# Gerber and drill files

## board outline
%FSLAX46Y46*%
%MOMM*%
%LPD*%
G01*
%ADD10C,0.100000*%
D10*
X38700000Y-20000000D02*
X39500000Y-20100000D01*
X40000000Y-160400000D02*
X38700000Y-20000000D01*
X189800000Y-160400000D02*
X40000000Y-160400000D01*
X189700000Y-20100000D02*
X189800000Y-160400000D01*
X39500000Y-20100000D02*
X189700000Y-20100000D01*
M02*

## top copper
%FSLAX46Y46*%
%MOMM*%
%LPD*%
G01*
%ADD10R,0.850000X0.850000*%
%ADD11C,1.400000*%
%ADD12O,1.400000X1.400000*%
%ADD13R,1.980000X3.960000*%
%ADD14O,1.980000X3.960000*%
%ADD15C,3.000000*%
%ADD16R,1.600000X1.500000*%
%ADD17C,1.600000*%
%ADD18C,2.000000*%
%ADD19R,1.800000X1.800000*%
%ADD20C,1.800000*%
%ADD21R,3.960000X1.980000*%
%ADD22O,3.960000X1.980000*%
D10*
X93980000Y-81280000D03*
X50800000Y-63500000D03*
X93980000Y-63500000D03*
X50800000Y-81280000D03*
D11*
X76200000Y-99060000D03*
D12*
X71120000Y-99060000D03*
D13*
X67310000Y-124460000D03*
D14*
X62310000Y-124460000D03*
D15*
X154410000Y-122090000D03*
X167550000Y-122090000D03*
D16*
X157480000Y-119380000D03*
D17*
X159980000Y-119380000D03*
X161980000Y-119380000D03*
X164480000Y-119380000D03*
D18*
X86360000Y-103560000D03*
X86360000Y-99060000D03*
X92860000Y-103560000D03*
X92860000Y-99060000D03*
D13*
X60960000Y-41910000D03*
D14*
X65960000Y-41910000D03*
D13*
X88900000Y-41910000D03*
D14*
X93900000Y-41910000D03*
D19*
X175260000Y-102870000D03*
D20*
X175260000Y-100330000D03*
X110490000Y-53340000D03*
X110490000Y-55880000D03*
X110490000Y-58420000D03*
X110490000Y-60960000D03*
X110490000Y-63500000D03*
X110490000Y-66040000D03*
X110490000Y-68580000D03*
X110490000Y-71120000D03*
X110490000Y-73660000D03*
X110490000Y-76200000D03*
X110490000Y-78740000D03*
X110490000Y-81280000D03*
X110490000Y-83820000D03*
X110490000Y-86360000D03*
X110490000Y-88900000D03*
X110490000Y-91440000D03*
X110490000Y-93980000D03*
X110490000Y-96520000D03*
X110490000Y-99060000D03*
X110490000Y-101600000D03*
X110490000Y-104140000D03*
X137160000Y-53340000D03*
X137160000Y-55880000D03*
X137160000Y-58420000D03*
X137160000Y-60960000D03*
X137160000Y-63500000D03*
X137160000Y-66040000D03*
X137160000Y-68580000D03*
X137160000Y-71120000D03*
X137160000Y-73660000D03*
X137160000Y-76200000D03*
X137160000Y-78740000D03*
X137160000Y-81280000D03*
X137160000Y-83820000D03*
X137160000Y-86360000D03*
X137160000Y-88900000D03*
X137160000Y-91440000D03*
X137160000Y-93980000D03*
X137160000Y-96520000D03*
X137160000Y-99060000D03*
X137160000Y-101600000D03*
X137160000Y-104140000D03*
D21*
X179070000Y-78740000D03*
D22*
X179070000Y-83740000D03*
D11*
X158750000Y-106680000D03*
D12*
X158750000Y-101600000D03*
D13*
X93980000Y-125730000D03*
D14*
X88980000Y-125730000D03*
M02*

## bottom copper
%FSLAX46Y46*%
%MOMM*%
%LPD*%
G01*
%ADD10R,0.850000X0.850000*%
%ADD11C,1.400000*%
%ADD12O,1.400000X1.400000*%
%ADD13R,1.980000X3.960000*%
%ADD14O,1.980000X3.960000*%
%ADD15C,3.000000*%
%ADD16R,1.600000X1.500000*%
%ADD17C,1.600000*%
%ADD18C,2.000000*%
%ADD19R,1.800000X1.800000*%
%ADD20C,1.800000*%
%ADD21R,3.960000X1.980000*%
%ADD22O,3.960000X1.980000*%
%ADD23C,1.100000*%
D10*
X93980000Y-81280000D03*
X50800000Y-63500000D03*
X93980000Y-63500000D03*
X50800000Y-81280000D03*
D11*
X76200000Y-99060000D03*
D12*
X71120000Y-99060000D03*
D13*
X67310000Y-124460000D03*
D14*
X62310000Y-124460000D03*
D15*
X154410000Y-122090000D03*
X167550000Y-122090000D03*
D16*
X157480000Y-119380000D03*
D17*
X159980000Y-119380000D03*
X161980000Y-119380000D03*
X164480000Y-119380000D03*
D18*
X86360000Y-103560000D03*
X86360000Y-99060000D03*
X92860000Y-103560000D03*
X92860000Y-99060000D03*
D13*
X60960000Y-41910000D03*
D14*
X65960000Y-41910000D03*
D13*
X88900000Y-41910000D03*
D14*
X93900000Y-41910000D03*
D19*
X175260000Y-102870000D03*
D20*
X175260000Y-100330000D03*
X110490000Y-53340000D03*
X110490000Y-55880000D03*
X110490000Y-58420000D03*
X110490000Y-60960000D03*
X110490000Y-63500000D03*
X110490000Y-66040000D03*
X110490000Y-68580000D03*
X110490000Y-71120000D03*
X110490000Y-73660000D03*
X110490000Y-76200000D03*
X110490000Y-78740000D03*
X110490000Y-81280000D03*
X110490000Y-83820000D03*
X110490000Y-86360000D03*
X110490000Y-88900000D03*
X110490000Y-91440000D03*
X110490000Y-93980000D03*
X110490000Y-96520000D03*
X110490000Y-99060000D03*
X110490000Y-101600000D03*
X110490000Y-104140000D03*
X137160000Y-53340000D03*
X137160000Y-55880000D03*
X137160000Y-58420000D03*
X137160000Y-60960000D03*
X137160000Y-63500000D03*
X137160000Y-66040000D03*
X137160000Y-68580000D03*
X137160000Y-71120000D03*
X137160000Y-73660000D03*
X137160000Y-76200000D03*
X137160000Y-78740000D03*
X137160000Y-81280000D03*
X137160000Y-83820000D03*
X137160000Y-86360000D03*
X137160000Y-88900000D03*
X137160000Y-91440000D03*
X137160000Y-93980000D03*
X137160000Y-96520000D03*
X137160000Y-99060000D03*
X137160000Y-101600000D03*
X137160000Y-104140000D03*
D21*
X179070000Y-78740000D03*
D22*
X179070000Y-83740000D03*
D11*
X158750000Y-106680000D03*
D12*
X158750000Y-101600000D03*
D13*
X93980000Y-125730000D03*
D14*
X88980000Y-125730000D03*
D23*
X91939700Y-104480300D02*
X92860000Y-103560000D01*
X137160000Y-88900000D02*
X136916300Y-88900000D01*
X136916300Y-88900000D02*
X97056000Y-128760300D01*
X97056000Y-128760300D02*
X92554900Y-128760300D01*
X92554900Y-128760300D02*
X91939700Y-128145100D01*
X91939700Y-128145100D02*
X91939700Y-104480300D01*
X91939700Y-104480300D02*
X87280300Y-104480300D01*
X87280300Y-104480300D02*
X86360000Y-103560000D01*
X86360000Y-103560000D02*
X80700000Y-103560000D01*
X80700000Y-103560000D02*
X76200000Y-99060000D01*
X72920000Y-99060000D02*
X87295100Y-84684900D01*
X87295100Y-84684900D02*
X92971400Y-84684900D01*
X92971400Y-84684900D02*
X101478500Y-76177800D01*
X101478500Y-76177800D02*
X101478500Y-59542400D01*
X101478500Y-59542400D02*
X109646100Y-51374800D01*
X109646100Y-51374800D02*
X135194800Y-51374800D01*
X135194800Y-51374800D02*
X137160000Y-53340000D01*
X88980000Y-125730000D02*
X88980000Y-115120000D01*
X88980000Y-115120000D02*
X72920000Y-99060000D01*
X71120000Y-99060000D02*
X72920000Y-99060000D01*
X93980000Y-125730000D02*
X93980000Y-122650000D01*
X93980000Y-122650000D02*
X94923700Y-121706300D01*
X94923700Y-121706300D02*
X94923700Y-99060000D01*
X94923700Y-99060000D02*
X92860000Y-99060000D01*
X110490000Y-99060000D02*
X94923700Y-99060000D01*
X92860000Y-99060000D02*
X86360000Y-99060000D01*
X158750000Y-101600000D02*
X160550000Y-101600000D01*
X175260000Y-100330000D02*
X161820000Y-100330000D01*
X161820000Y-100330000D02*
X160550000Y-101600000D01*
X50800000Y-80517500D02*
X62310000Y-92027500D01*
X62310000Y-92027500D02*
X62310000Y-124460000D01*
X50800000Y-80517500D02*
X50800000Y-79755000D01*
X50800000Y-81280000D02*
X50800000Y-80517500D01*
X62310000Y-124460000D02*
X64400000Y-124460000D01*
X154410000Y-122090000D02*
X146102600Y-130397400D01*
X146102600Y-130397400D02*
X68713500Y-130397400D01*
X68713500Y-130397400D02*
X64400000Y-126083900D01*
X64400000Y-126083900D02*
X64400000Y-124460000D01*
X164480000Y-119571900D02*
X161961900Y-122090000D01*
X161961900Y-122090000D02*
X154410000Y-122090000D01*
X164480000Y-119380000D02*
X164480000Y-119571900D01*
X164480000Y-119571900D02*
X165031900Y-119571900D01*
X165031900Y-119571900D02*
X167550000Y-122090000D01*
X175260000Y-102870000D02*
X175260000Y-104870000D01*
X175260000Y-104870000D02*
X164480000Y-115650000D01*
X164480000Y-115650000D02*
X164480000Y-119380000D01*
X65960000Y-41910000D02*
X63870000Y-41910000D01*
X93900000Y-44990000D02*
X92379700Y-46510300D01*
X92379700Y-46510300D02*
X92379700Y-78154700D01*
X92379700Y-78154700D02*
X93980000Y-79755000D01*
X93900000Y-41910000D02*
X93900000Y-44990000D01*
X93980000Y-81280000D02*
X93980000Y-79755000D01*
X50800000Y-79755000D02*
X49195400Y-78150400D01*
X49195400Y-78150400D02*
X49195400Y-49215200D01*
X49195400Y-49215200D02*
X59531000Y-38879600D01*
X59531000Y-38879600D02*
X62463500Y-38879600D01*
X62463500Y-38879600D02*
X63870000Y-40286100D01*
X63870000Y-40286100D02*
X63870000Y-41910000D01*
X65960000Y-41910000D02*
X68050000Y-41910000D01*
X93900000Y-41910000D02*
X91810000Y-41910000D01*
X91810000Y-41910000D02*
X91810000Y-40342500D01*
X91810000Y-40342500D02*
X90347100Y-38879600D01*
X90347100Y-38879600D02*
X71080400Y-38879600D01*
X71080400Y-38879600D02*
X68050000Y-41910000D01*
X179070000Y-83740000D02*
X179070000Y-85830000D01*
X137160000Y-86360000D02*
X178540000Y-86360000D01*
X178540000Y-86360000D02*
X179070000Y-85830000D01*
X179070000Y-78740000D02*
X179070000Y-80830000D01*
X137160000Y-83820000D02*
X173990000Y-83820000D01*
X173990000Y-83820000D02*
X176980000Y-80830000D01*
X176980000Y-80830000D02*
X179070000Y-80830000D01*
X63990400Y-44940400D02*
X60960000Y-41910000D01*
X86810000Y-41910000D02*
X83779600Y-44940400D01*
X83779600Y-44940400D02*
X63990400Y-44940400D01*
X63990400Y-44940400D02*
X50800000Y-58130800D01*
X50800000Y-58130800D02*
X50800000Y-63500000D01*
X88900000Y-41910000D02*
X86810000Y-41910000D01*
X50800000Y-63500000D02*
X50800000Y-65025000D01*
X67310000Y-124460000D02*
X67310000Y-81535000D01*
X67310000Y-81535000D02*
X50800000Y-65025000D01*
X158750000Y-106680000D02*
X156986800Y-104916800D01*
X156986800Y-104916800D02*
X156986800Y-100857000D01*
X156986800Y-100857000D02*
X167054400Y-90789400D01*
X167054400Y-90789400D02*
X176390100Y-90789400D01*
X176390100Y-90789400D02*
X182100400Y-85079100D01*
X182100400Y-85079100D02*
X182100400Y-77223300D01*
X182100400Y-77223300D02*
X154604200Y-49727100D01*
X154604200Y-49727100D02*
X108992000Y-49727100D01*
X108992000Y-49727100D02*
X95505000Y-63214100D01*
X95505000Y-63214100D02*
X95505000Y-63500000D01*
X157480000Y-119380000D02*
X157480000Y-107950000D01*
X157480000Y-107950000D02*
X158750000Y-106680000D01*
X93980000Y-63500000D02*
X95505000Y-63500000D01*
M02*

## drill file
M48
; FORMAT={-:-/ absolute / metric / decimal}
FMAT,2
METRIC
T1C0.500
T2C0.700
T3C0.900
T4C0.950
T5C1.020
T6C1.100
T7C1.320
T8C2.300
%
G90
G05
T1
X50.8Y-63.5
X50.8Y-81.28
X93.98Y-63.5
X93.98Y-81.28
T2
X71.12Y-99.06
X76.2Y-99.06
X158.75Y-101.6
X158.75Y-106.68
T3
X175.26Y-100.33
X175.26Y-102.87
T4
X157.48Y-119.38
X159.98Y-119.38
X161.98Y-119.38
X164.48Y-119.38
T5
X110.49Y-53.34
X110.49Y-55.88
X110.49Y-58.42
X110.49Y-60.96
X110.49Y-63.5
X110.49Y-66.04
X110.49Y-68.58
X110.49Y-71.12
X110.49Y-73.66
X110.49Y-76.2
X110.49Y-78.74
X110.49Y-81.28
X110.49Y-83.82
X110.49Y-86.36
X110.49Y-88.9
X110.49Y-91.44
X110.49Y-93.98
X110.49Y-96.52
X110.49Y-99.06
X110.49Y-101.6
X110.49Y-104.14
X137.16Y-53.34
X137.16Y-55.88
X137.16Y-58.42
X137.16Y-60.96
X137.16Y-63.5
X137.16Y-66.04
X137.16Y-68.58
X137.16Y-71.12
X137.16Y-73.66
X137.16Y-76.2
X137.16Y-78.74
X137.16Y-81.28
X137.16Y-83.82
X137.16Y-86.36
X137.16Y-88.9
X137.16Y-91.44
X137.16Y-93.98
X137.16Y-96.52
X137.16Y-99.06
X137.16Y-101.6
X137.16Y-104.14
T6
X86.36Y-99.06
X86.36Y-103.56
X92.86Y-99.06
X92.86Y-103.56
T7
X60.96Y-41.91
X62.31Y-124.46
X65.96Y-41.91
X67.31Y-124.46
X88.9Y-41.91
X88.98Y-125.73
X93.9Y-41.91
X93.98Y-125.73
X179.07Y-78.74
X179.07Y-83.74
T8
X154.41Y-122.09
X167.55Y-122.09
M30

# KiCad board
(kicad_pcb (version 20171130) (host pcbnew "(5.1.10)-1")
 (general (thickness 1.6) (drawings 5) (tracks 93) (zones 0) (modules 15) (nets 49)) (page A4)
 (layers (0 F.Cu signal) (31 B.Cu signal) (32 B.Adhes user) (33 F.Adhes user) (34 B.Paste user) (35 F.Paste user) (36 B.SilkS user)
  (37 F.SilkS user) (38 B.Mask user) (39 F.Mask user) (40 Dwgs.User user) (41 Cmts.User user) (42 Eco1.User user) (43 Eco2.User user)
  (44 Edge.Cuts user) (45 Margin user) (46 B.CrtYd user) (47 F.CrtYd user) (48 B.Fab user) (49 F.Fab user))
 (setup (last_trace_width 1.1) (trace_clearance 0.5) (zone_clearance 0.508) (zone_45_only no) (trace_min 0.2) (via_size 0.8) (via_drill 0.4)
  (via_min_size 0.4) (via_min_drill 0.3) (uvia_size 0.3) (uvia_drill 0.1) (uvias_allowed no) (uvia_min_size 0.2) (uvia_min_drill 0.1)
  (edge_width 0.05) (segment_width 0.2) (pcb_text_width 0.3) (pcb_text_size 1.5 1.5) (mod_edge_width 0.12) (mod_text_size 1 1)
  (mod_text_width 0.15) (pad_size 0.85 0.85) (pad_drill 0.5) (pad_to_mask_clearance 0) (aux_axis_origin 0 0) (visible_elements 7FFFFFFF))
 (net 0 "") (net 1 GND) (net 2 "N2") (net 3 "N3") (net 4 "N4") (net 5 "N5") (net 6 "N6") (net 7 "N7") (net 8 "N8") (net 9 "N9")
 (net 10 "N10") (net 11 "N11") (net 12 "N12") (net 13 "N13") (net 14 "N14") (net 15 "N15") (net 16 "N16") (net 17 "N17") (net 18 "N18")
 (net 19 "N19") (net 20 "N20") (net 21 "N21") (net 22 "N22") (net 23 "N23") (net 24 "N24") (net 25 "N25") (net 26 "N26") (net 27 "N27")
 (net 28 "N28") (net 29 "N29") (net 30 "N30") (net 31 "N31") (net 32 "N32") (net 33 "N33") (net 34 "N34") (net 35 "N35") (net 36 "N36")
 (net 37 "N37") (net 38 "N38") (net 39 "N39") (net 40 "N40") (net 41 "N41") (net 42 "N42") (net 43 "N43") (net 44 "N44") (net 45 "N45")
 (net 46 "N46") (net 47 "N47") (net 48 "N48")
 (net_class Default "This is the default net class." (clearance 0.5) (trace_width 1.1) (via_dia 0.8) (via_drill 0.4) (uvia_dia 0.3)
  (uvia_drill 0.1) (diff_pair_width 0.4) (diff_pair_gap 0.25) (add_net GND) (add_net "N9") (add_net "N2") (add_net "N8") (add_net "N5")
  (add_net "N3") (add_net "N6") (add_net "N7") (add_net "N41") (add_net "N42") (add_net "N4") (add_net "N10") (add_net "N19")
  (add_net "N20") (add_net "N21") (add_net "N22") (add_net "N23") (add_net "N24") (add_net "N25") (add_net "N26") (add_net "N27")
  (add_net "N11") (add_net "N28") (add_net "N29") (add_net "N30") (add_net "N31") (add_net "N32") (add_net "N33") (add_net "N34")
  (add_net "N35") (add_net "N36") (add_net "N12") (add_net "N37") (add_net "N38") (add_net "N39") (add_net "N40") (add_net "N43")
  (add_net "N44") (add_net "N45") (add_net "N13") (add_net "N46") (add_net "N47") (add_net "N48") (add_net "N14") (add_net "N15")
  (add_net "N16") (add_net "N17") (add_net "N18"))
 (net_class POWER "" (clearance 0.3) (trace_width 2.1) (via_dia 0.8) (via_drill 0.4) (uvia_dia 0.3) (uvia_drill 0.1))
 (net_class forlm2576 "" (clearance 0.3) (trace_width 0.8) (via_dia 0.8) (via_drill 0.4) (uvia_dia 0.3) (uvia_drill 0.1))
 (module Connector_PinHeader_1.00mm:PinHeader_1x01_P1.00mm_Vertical (layer F.Cu) (at 93.98 81.28)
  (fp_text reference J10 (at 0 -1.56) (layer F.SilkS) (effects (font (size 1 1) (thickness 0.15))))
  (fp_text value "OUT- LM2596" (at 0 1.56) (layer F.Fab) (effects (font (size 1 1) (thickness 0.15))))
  (pad 1 thru_hole rect (at 0 0) (size 0.85 0.85) (drill 0.5) (layers *.Cu *.Mask) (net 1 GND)))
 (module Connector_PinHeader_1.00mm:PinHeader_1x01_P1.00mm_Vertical (layer F.Cu) (at 50.8 63.5)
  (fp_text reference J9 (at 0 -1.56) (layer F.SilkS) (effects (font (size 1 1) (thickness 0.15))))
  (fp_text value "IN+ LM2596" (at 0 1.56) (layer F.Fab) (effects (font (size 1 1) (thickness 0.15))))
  (pad 1 thru_hole rect (at 0 0) (size 0.85 0.85) (drill 0.5) (layers *.Cu *.Mask) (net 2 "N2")))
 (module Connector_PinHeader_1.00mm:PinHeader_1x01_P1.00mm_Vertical (layer F.Cu) (at 93.98 63.5)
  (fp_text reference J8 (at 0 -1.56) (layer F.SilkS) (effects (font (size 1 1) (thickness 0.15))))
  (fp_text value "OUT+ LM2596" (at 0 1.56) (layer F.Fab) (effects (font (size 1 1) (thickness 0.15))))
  (pad 1 thru_hole rect (at 0 0) (size 0.85 0.85) (drill 0.5) (layers *.Cu *.Mask) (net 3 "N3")))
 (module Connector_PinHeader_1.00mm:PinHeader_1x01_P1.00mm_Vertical (layer F.Cu) (at 50.8 81.28)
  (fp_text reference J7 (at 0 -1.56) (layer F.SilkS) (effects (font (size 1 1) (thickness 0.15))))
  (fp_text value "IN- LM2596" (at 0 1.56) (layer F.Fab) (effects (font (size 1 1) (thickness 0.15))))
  (pad 1 thru_hole rect (at 0 0) (size 0.85 0.85) (drill 0.5) (layers *.Cu *.Mask) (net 1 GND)))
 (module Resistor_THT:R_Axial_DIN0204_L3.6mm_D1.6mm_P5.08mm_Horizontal (layer F.Cu) (at 76.2 99.06 180)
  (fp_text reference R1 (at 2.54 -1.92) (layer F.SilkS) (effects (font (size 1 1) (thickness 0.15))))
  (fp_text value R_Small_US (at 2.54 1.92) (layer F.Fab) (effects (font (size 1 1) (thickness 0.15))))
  (pad 1 thru_hole circle (at 0 0 180) (size 1.4 1.4) (drill 0.7) (layers *.Cu *.Mask) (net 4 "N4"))
  (pad 2 thru_hole oval (at 5.08 0 180) (size 1.4 1.4) (drill 0.7) (layers *.Cu *.Mask) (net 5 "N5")))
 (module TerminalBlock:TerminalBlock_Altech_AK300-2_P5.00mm (layer F.Cu) (at 67.31 124.46 180)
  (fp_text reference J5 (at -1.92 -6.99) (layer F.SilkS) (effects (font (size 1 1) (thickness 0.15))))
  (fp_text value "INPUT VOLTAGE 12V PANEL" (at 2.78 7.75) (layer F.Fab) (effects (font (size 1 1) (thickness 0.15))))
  (pad 1 thru_hole rect (at 0 0 180) (size 1.98 3.96) (drill 1.32) (layers *.Cu *.Mask) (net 2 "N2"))
  (pad 2 thru_hole oval (at 5 0 180) (size 1.98 3.96) (drill 1.32) (layers *.Cu *.Mask) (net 1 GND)))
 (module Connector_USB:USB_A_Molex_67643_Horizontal (layer F.Cu) (at 157.48 119.38)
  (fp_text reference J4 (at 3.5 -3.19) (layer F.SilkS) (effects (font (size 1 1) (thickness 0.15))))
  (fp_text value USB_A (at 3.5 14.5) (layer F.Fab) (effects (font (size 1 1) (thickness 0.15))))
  (pad 5 thru_hole circle (at -3.07 2.71) (size 3 3) (drill 2.3) (layers *.Cu *.Mask) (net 1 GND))
  (pad 5 thru_hole circle (at 10.07 2.71) (size 3 3) (drill 2.3) (layers *.Cu *.Mask) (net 1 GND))
  (pad 1 thru_hole rect (at 0 0) (size 1.6 1.5) (drill 0.95) (layers *.Cu *.Mask) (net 3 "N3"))
  (pad 2 thru_hole circle (at 2.5 0) (size 1.6 1.6) (drill 0.95) (layers *.Cu *.Mask) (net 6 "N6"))
  (pad 3 thru_hole circle (at 4.5 0) (size 1.6 1.6) (drill 0.95) (layers *.Cu *.Mask) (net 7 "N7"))
  (pad 4 thru_hole circle (at 7 0) (size 1.6 1.6) (drill 0.95) (layers *.Cu *.Mask) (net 1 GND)))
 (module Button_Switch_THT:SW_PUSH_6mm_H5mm (layer F.Cu) (at 86.36 99.06)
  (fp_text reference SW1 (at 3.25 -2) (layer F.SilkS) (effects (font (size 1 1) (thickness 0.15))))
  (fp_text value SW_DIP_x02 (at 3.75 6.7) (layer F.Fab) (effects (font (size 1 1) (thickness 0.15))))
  (pad 2 thru_hole circle (at 0 4.5 90) (size 2 2) (drill 1.1) (layers *.Cu *.Mask) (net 4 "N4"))
  (pad 1 thru_hole circle (at 0 0 90) (size 2 2) (drill 1.1) (layers *.Cu *.Mask) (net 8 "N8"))
  (pad 2 thru_hole circle (at 6.5 4.5 90) (size 2 2) (drill 1.1) (layers *.Cu *.Mask) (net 4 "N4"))
  (pad 1 thru_hole circle (at 6.5 0 90) (size 2 2) (drill 1.1) (layers *.Cu *.Mask) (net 8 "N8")))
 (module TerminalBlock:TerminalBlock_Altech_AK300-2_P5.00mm (layer F.Cu) (at 60.96 41.91)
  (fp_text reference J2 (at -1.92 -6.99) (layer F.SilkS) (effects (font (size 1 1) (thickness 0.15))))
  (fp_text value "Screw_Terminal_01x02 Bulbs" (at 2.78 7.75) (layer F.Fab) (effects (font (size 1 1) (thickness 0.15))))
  (pad 1 thru_hole rect (at 0 0) (size 1.98 3.96) (drill 1.32) (layers *.Cu *.Mask) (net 2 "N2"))
  (pad 2 thru_hole oval (at 5 0) (size 1.98 3.96) (drill 1.32) (layers *.Cu *.Mask) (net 1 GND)))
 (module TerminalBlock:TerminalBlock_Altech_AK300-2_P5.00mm (layer F.Cu) (at 88.9 41.91)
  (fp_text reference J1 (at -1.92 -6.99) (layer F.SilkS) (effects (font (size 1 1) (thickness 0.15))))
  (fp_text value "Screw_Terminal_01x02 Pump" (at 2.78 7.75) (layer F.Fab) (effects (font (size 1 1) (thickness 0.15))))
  (pad 1 thru_hole rect (at 0 0) (size 1.98 3.96) (drill 1.32) (layers *.Cu *.Mask) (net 2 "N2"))
  (pad 2 thru_hole oval (at 5 0) (size 1.98 3.96) (drill 1.32) (layers *.Cu *.Mask) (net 1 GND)))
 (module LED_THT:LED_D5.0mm (layer F.Cu) (at 175.26 102.87 90)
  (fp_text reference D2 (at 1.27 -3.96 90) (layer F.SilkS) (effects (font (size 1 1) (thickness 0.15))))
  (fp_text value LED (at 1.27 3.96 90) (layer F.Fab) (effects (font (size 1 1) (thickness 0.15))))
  (pad 1 thru_hole rect (at 0 0 90) (size 1.8 1.8) (drill 0.9) (layers *.Cu *.Mask) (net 1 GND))
  (pad 2 thru_hole circle (at 2.54 0 90) (size 1.8 1.8) (drill 0.9) (layers *.Cu *.Mask) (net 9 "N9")))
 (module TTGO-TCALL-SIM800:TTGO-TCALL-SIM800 (layer F.Cu) (at 110.49 53.34)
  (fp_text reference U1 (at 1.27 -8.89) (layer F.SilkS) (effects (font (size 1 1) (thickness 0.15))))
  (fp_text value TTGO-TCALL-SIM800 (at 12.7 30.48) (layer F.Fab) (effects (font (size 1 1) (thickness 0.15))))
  (pad 1 thru_hole circle (at 0 0) (size 1.8 1.8) (drill 1.02) (layers *.Cu *.Mask) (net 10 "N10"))
  (pad 2 thru_hole circle (at 0 2.54) (size 1.8 1.8) (drill 1.02) (layers *.Cu *.Mask) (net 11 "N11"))
  (pad 3 thru_hole circle (at 0 5.08) (size 1.8 1.8) (drill 1.02) (layers *.Cu *.Mask) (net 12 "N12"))
  (pad 4 thru_hole circle (at 0 7.62) (size 1.8 1.8) (drill 1.02) (layers *.Cu *.Mask) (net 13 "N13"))
  (pad 5 thru_hole circle (at 0 10.16) (size 1.8 1.8) (drill 1.02) (layers *.Cu *.Mask) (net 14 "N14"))
  (pad 6 thru_hole circle (at 0 12.7) (size 1.8 1.8) (drill 1.02) (layers *.Cu *.Mask) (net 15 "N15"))
  (pad 7 thru_hole circle (at 0 15.24) (size 1.8 1.8) (drill 1.02) (layers *.Cu *.Mask) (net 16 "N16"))
  (pad 8 thru_hole circle (at 0 17.78) (size 1.8 1.8) (drill 1.02) (layers *.Cu *.Mask) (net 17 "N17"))
  (pad 9 thru_hole circle (at 0 20.32) (size 1.8 1.8) (drill 1.02) (layers *.Cu *.Mask) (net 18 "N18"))
  (pad 10 thru_hole circle (at 0 22.86) (size 1.8 1.8) (drill 1.02) (layers *.Cu *.Mask) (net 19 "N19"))
  (pad 11 thru_hole circle (at 0 25.4) (size 1.8 1.8) (drill 1.02) (layers *.Cu *.Mask) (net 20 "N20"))
  (pad 12 thru_hole circle (at 0 27.94) (size 1.8 1.8) (drill 1.02) (layers *.Cu *.Mask) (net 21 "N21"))
  (pad 13 thru_hole circle (at 0 30.48) (size 1.8 1.8) (drill 1.02) (layers *.Cu *.Mask) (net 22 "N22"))
  (pad 14 thru_hole circle (at 0 33.02) (size 1.8 1.8) (drill 1.02) (layers *.Cu *.Mask) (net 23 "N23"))
  (pad 15 thru_hole circle (at 0 35.56) (size 1.8 1.8) (drill 1.02) (layers *.Cu *.Mask) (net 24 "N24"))
  (pad 16 thru_hole circle (at 0 38.1) (size 1.8 1.8) (drill 1.02) (layers *.Cu *.Mask) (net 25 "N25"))
  (pad 17 thru_hole circle (at 0 40.64) (size 1.8 1.8) (drill 1.02) (layers *.Cu *.Mask) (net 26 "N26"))
  (pad 18 thru_hole circle (at 0 43.18) (size 1.8 1.8) (drill 1.02) (layers *.Cu *.Mask) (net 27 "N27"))
  (pad 19 thru_hole circle (at 0 45.72) (size 1.8 1.8) (drill 1.02) (layers *.Cu *.Mask) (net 8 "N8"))
  (pad 20 thru_hole circle (at 0 48.26) (size 1.8 1.8) (drill 1.02) (layers *.Cu *.Mask) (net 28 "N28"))
  (pad 21 thru_hole circle (at 0 50.8) (size 1.8 1.8) (drill 1.02) (layers *.Cu *.Mask) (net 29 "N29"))
  (pad 22 thru_hole circle (at 26.67 0) (size 1.8 1.8) (drill 1.02) (layers *.Cu *.Mask) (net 5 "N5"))
  (pad 23 thru_hole circle (at 26.67 2.54) (size 1.8 1.8) (drill 1.02) (layers *.Cu *.Mask) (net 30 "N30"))
  (pad 24 thru_hole circle (at 26.67 5.08) (size 1.8 1.8) (drill 1.02) (layers *.Cu *.Mask) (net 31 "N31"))
  (pad 25 thru_hole circle (at 26.67 7.62) (size 1.8 1.8) (drill 1.02) (layers *.Cu *.Mask) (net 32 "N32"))
  (pad 26 thru_hole circle (at 26.67 10.16) (size 1.8 1.8) (drill 1.02) (layers *.Cu *.Mask) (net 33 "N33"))
  (pad 27 thru_hole circle (at 26.67 12.7) (size 1.8 1.8) (drill 1.02) (layers *.Cu *.Mask) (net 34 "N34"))
  (pad 28 thru_hole circle (at 26.67 15.24) (size 1.8 1.8) (drill 1.02) (layers *.Cu *.Mask) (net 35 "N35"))
  (pad 29 thru_hole circle (at 26.67 17.78) (size 1.8 1.8) (drill 1.02) (layers *.Cu *.Mask) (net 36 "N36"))
  (pad 30 thru_hole circle (at 26.67 20.32) (size 1.8 1.8) (drill 1.02) (layers *.Cu *.Mask) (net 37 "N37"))
  (pad 31 thru_hole circle (at 26.67 22.86) (size 1.8 1.8) (drill 1.02) (layers *.Cu *.Mask) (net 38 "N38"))
  (pad 32 thru_hole circle (at 26.67 25.4) (size 1.8 1.8) (drill 1.02) (layers *.Cu *.Mask) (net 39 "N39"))
  (pad 33 thru_hole circle (at 26.67 27.94) (size 1.8 1.8) (drill 1.02) (layers *.Cu *.Mask) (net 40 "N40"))
  (pad 34 thru_hole circle (at 26.67 30.48) (size 1.8 1.8) (drill 1.02) (layers *.Cu *.Mask) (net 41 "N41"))
  (pad 35 thru_hole circle (at 26.67 33.02) (size 1.8 1.8) (drill 1.02) (layers *.Cu *.Mask) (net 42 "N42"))
  (pad 36 thru_hole circle (at 26.67 35.56) (size 1.8 1.8) (drill 1.02) (layers *.Cu *.Mask) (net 4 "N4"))
  (pad 37 thru_hole circle (at 26.67 38.1) (size 1.8 1.8) (drill 1.02) (layers *.Cu *.Mask) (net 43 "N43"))
  (pad 38 thru_hole circle (at 26.67 40.64) (size 1.8 1.8) (drill 1.02) (layers *.Cu *.Mask) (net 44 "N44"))
  (pad 39 thru_hole circle (at 26.67 43.18) (size 1.8 1.8) (drill 1.02) (layers *.Cu *.Mask) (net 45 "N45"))
  (pad 40 thru_hole circle (at 26.67 45.72) (size 1.8 1.8) (drill 1.02) (layers *.Cu *.Mask) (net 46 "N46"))
  (pad 41 thru_hole circle (at 26.67 48.26) (size 1.8 1.8) (drill 1.02) (layers *.Cu *.Mask) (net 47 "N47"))
  (pad 42 thru_hole circle (at 26.67 50.8) (size 1.8 1.8) (drill 1.02) (layers *.Cu *.Mask) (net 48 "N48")))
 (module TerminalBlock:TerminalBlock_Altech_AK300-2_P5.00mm (layer F.Cu) (at 179.07 78.74 270)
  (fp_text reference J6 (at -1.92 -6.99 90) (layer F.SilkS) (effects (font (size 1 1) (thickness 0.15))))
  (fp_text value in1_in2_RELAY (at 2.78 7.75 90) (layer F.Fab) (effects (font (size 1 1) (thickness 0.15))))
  (pad 1 thru_hole rect (at 0 0 270) (size 1.98 3.96) (drill 1.32) (layers *.Cu *.Mask) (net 41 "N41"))
  (pad 2 thru_hole oval (at 5 0 270) (size 1.98 3.96) (drill 1.32) (layers *.Cu *.Mask) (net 42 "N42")))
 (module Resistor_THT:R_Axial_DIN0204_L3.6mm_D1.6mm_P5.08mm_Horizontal (layer F.Cu) (at 158.75 106.68 90)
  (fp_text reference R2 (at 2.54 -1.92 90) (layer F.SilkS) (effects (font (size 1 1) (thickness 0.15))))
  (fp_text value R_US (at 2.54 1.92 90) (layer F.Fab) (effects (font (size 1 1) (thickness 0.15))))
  (pad 1 thru_hole circle (at 0 0 90) (size 1.4 1.4) (drill 0.7) (layers *.Cu *.Mask) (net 3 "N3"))
  (pad 2 thru_hole oval (at 5.08 0 90) (size 1.4 1.4) (drill 0.7) (layers *.Cu *.Mask) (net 9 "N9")))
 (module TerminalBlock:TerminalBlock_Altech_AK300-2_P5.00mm (layer F.Cu) (at 93.98 125.73 180)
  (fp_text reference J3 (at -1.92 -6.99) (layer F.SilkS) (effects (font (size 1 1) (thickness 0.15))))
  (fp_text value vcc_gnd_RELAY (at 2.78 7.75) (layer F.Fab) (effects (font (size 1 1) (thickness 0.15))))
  (pad 1 thru_hole rect (at 0 0 180) (size 1.98 3.96) (drill 1.32) (layers *.Cu *.Mask) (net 8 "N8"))
  (pad 2 thru_hole oval (at 5 0 180) (size 1.98 3.96) (drill 1.32) (layers *.Cu *.Mask) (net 5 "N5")))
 (gr_line (start 38.7 20) (end 39.5 20.1) (layer Edge.Cuts) (width 0.1))
 (gr_line (start 40 160.4) (end 38.7 20) (layer Edge.Cuts) (width 0.1))
 (gr_line (start 189.8 160.4) (end 40 160.4) (layer Edge.Cuts) (width 0.1))
 (gr_line (start 189.7 20.1) (end 189.8 160.4) (layer Edge.Cuts) (width 0.1))
 (gr_line (start 39.5 20.1) (end 189.7 20.1) (layer Edge.Cuts) (width 0.1))
 (segment (start 91.9397 104.4803) (end 92.86 103.56) (width 1.1) (layer B.Cu) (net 4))
 (segment (start 137.16 88.9) (end 136.9163 88.9) (width 1.1) (layer B.Cu) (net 4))
 (segment (start 136.9163 88.9) (end 97.056 128.7603) (width 1.1) (layer B.Cu) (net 4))
 (segment (start 97.056 128.7603) (end 92.5549 128.7603) (width 1.1) (layer B.Cu) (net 4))
 (segment (start 92.5549 128.7603) (end 91.9397 128.1451) (width 1.1) (layer B.Cu) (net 4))
 (segment (start 91.9397 128.1451) (end 91.9397 104.4803) (width 1.1) (layer B.Cu) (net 4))
 (segment (start 91.9397 104.4803) (end 87.2803 104.4803) (width 1.1) (layer B.Cu) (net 4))
 (segment (start 87.2803 104.4803) (end 86.36 103.56) (width 1.1) (layer B.Cu) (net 4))
 (segment (start 86.36 103.56) (end 80.7 103.56) (width 1.1) (layer B.Cu) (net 4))
 (segment (start 80.7 103.56) (end 76.2 99.06) (width 1.1) (layer B.Cu) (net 4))
 (segment (start 72.92 99.06) (end 87.2951 84.6849) (width 1.1) (layer B.Cu) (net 5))
 (segment (start 87.2951 84.6849) (end 92.9714 84.6849) (width 1.1) (layer B.Cu) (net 5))
 (segment (start 92.9714 84.6849) (end 101.4785 76.1778) (width 1.1) (layer B.Cu) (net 5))
 (segment (start 101.4785 76.1778) (end 101.4785 59.5424) (width 1.1) (layer B.Cu) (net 5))
 (segment (start 101.4785 59.5424) (end 109.6461 51.3748) (width 1.1) (layer B.Cu) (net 5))
 (segment (start 109.6461 51.3748) (end 135.1948 51.3748) (width 1.1) (layer B.Cu) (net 5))
 (segment (start 135.1948 51.3748) (end 137.16 53.34) (width 1.1) (layer B.Cu) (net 5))
 (segment (start 88.98 125.73) (end 88.98 115.12) (width 1.1) (layer B.Cu) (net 5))
 (segment (start 88.98 115.12) (end 72.92 99.06) (width 1.1) (layer B.Cu) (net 5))
 (segment (start 71.12 99.06) (end 72.92 99.06) (width 1.1) (layer B.Cu) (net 5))
 (segment (start 93.98 125.73) (end 93.98 122.65) (width 1.1) (layer B.Cu) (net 8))
 (segment (start 93.98 122.65) (end 94.9237 121.7063) (width 1.1) (layer B.Cu) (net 8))
 (segment (start 94.9237 121.7063) (end 94.9237 99.06) (width 1.1) (layer B.Cu) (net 8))
 (segment (start 94.9237 99.06) (end 92.86 99.06) (width 1.1) (layer B.Cu) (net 8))
 (segment (start 110.49 99.06) (end 94.9237 99.06) (width 1.1) (layer B.Cu) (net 8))
 (segment (start 92.86 99.06) (end 86.36 99.06) (width 1.1) (layer B.Cu) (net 8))
 (segment (start 158.75 101.6) (end 160.55 101.6) (width 1.1) (layer B.Cu) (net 9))
 (segment (start 175.26 100.33) (end 161.82 100.33) (width 1.1) (layer B.Cu) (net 9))
 (segment (start 161.82 100.33) (end 160.55 101.6) (width 1.1) (layer B.Cu) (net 9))
 (segment (start 50.8 80.5175) (end 62.31 92.0275) (width 1.1) (layer B.Cu) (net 1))
 (segment (start 62.31 92.0275) (end 62.31 124.46) (width 1.1) (layer B.Cu) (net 1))
 (segment (start 50.8 80.5175) (end 50.8 79.755) (width 1.1) (layer B.Cu) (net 1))
 (segment (start 50.8 81.28) (end 50.8 80.5175) (width 1.1) (layer B.Cu) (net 1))
 (segment (start 62.31 124.46) (end 64.4 124.46) (width 1.1) (layer B.Cu) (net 1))
 (segment (start 154.41 122.09) (end 146.1026 130.3974) (width 1.1) (layer B.Cu) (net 1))
 (segment (start 146.1026 130.3974) (end 68.7135 130.3974) (width 1.1) (layer B.Cu) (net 1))
 (segment (start 68.7135 130.3974) (end 64.4 126.0839) (width 1.1) (layer B.Cu) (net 1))
 (segment (start 64.4 126.0839) (end 64.4 124.46) (width 1.1) (layer B.Cu) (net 1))
 (segment (start 164.48 119.5719) (end 161.9619 122.09) (width 1.1) (layer B.Cu) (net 1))
 (segment (start 161.9619 122.09) (end 154.41 122.09) (width 1.1) (layer B.Cu) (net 1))
 (segment (start 164.48 119.38) (end 164.48 119.5719) (width 1.1) (layer B.Cu) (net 1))
 (segment (start 164.48 119.5719) (end 165.0319 119.5719) (width 1.1) (layer B.Cu) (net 1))
 (segment (start 165.0319 119.5719) (end 167.55 122.09) (width 1.1) (layer B.Cu) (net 1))
 (segment (start 175.26 102.87) (end 175.26 104.87) (width 1.1) (layer B.Cu) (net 1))
 (segment (start 175.26 104.87) (end 164.48 115.65) (width 1.1) (layer B.Cu) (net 1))
 (segment (start 164.48 115.65) (end 164.48 119.38) (width 1.1) (layer B.Cu) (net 1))
 (segment (start 65.96 41.91) (end 63.87 41.91) (width 1.1) (layer B.Cu) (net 1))
 (segment (start 93.9 44.99) (end 92.3797 46.5103) (width 1.1) (layer B.Cu) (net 1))
 (segment (start 92.3797 46.5103) (end 92.3797 78.1547) (width 1.1) (layer B.Cu) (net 1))
 (segment (start 92.3797 78.1547) (end 93.98 79.755) (width 1.1) (layer B.Cu) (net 1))
 (segment (start 93.9 41.91) (end 93.9 44.99) (width 1.1) (layer B.Cu) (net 1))
 (segment (start 93.98 81.28) (end 93.98 79.755) (width 1.1) (layer B.Cu) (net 1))
 (segment (start 50.8 79.755) (end 49.1954 78.1504) (width 1.1) (layer B.Cu) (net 1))
 (segment (start 49.1954 78.1504) (end 49.1954 49.2152) (width 1.1) (layer B.Cu) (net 1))
 (segment (start 49.1954 49.2152) (end 59.531 38.8796) (width 1.1) (layer B.Cu) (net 1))
 (segment (start 59.531 38.8796) (end 62.4635 38.8796) (width 1.1) (layer B.Cu) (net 1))
 (segment (start 62.4635 38.8796) (end 63.87 40.2861) (width 1.1) (layer B.Cu) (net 1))
 (segment (start 63.87 40.2861) (end 63.87 41.91) (width 1.1) (layer B.Cu) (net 1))
 (segment (start 65.96 41.91) (end 68.05 41.91) (width 1.1) (layer B.Cu) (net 1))
 (segment (start 93.9 41.91) (end 91.81 41.91) (width 1.1) (layer B.Cu) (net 1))
 (segment (start 91.81 41.91) (end 91.81 40.3425) (width 1.1) (layer B.Cu) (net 1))
 (segment (start 91.81 40.3425) (end 90.3471 38.8796) (width 1.1) (layer B.Cu) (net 1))
 (segment (start 90.3471 38.8796) (end 71.0804 38.8796) (width 1.1) (layer B.Cu) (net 1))
 (segment (start 71.0804 38.8796) (end 68.05 41.91) (width 1.1) (layer B.Cu) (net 1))
 (segment (start 179.07 83.74) (end 179.07 85.83) (width 1.1) (layer B.Cu) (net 42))
 (segment (start 137.16 86.36) (end 178.54 86.36) (width 1.1) (layer B.Cu) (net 42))
 (segment (start 178.54 86.36) (end 179.07 85.83) (width 1.1) (layer B.Cu) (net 42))
 (segment (start 179.07 78.74) (end 179.07 80.83) (width 1.1) (layer B.Cu) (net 41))
 (segment (start 137.16 83.82) (end 173.99 83.82) (width 1.1) (layer B.Cu) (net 41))
 (segment (start 173.99 83.82) (end 176.98 80.83) (width 1.1) (layer B.Cu) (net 41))
 (segment (start 176.98 80.83) (end 179.07 80.83) (width 1.1) (layer B.Cu) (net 41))
 (segment (start 63.9904 44.9404) (end 60.96 41.91) (width 1.1) (layer B.Cu) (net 2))
 (segment (start 86.81 41.91) (end 83.7796 44.9404) (width 1.1) (layer B.Cu) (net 2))
 (segment (start 83.7796 44.9404) (end 63.9904 44.9404) (width 1.1) (layer B.Cu) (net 2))
 (segment (start 63.9904 44.9404) (end 50.8 58.1308) (width 1.1) (layer B.Cu) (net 2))
 (segment (start 50.8 58.1308) (end 50.8 63.5) (width 1.1) (layer B.Cu) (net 2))
 (segment (start 88.9 41.91) (end 86.81 41.91) (width 1.1) (layer B.Cu) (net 2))
 (segment (start 50.8 63.5) (end 50.8 65.025) (width 1.1) (layer B.Cu) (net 2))
 (segment (start 67.31 124.46) (end 67.31 81.535) (width 1.1) (layer B.Cu) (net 2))
 (segment (start 67.31 81.535) (end 50.8 65.025) (width 1.1) (layer B.Cu) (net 2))
 (segment (start 158.75 106.68) (end 156.9868 104.9168) (width 1.1) (layer B.Cu) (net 3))
 (segment (start 156.9868 104.9168) (end 156.9868 100.857) (width 1.1) (layer B.Cu) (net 3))
 (segment (start 156.9868 100.857) (end 167.0544 90.7894) (width 1.1) (layer B.Cu) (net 3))
 (segment (start 167.0544 90.7894) (end 176.3901 90.7894) (width 1.1) (layer B.Cu) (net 3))
 (segment (start 176.3901 90.7894) (end 182.1004 85.0791) (width 1.1) (layer B.Cu) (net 3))
 (segment (start 182.1004 85.0791) (end 182.1004 77.2233) (width 1.1) (layer B.Cu) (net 3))
 (segment (start 182.1004 77.2233) (end 154.6042 49.7271) (width 1.1) (layer B.Cu) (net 3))
 (segment (start 154.6042 49.7271) (end 108.992 49.7271) (width 1.1) (layer B.Cu) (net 3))
 (segment (start 108.992 49.7271) (end 95.505 63.2141) (width 1.1) (layer B.Cu) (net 3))
 (segment (start 95.505 63.2141) (end 95.505 63.5) (width 1.1) (layer B.Cu) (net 3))
 (segment (start 157.48 119.38) (end 157.48 107.95) (width 1.1) (layer B.Cu) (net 3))
 (segment (start 157.48 107.95) (end 158.75 106.68) (width 1.1) (layer B.Cu) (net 3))
 (segment (start 93.98 63.5) (end 95.505 63.5) (width 1.1) (layer B.Cu) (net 3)))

